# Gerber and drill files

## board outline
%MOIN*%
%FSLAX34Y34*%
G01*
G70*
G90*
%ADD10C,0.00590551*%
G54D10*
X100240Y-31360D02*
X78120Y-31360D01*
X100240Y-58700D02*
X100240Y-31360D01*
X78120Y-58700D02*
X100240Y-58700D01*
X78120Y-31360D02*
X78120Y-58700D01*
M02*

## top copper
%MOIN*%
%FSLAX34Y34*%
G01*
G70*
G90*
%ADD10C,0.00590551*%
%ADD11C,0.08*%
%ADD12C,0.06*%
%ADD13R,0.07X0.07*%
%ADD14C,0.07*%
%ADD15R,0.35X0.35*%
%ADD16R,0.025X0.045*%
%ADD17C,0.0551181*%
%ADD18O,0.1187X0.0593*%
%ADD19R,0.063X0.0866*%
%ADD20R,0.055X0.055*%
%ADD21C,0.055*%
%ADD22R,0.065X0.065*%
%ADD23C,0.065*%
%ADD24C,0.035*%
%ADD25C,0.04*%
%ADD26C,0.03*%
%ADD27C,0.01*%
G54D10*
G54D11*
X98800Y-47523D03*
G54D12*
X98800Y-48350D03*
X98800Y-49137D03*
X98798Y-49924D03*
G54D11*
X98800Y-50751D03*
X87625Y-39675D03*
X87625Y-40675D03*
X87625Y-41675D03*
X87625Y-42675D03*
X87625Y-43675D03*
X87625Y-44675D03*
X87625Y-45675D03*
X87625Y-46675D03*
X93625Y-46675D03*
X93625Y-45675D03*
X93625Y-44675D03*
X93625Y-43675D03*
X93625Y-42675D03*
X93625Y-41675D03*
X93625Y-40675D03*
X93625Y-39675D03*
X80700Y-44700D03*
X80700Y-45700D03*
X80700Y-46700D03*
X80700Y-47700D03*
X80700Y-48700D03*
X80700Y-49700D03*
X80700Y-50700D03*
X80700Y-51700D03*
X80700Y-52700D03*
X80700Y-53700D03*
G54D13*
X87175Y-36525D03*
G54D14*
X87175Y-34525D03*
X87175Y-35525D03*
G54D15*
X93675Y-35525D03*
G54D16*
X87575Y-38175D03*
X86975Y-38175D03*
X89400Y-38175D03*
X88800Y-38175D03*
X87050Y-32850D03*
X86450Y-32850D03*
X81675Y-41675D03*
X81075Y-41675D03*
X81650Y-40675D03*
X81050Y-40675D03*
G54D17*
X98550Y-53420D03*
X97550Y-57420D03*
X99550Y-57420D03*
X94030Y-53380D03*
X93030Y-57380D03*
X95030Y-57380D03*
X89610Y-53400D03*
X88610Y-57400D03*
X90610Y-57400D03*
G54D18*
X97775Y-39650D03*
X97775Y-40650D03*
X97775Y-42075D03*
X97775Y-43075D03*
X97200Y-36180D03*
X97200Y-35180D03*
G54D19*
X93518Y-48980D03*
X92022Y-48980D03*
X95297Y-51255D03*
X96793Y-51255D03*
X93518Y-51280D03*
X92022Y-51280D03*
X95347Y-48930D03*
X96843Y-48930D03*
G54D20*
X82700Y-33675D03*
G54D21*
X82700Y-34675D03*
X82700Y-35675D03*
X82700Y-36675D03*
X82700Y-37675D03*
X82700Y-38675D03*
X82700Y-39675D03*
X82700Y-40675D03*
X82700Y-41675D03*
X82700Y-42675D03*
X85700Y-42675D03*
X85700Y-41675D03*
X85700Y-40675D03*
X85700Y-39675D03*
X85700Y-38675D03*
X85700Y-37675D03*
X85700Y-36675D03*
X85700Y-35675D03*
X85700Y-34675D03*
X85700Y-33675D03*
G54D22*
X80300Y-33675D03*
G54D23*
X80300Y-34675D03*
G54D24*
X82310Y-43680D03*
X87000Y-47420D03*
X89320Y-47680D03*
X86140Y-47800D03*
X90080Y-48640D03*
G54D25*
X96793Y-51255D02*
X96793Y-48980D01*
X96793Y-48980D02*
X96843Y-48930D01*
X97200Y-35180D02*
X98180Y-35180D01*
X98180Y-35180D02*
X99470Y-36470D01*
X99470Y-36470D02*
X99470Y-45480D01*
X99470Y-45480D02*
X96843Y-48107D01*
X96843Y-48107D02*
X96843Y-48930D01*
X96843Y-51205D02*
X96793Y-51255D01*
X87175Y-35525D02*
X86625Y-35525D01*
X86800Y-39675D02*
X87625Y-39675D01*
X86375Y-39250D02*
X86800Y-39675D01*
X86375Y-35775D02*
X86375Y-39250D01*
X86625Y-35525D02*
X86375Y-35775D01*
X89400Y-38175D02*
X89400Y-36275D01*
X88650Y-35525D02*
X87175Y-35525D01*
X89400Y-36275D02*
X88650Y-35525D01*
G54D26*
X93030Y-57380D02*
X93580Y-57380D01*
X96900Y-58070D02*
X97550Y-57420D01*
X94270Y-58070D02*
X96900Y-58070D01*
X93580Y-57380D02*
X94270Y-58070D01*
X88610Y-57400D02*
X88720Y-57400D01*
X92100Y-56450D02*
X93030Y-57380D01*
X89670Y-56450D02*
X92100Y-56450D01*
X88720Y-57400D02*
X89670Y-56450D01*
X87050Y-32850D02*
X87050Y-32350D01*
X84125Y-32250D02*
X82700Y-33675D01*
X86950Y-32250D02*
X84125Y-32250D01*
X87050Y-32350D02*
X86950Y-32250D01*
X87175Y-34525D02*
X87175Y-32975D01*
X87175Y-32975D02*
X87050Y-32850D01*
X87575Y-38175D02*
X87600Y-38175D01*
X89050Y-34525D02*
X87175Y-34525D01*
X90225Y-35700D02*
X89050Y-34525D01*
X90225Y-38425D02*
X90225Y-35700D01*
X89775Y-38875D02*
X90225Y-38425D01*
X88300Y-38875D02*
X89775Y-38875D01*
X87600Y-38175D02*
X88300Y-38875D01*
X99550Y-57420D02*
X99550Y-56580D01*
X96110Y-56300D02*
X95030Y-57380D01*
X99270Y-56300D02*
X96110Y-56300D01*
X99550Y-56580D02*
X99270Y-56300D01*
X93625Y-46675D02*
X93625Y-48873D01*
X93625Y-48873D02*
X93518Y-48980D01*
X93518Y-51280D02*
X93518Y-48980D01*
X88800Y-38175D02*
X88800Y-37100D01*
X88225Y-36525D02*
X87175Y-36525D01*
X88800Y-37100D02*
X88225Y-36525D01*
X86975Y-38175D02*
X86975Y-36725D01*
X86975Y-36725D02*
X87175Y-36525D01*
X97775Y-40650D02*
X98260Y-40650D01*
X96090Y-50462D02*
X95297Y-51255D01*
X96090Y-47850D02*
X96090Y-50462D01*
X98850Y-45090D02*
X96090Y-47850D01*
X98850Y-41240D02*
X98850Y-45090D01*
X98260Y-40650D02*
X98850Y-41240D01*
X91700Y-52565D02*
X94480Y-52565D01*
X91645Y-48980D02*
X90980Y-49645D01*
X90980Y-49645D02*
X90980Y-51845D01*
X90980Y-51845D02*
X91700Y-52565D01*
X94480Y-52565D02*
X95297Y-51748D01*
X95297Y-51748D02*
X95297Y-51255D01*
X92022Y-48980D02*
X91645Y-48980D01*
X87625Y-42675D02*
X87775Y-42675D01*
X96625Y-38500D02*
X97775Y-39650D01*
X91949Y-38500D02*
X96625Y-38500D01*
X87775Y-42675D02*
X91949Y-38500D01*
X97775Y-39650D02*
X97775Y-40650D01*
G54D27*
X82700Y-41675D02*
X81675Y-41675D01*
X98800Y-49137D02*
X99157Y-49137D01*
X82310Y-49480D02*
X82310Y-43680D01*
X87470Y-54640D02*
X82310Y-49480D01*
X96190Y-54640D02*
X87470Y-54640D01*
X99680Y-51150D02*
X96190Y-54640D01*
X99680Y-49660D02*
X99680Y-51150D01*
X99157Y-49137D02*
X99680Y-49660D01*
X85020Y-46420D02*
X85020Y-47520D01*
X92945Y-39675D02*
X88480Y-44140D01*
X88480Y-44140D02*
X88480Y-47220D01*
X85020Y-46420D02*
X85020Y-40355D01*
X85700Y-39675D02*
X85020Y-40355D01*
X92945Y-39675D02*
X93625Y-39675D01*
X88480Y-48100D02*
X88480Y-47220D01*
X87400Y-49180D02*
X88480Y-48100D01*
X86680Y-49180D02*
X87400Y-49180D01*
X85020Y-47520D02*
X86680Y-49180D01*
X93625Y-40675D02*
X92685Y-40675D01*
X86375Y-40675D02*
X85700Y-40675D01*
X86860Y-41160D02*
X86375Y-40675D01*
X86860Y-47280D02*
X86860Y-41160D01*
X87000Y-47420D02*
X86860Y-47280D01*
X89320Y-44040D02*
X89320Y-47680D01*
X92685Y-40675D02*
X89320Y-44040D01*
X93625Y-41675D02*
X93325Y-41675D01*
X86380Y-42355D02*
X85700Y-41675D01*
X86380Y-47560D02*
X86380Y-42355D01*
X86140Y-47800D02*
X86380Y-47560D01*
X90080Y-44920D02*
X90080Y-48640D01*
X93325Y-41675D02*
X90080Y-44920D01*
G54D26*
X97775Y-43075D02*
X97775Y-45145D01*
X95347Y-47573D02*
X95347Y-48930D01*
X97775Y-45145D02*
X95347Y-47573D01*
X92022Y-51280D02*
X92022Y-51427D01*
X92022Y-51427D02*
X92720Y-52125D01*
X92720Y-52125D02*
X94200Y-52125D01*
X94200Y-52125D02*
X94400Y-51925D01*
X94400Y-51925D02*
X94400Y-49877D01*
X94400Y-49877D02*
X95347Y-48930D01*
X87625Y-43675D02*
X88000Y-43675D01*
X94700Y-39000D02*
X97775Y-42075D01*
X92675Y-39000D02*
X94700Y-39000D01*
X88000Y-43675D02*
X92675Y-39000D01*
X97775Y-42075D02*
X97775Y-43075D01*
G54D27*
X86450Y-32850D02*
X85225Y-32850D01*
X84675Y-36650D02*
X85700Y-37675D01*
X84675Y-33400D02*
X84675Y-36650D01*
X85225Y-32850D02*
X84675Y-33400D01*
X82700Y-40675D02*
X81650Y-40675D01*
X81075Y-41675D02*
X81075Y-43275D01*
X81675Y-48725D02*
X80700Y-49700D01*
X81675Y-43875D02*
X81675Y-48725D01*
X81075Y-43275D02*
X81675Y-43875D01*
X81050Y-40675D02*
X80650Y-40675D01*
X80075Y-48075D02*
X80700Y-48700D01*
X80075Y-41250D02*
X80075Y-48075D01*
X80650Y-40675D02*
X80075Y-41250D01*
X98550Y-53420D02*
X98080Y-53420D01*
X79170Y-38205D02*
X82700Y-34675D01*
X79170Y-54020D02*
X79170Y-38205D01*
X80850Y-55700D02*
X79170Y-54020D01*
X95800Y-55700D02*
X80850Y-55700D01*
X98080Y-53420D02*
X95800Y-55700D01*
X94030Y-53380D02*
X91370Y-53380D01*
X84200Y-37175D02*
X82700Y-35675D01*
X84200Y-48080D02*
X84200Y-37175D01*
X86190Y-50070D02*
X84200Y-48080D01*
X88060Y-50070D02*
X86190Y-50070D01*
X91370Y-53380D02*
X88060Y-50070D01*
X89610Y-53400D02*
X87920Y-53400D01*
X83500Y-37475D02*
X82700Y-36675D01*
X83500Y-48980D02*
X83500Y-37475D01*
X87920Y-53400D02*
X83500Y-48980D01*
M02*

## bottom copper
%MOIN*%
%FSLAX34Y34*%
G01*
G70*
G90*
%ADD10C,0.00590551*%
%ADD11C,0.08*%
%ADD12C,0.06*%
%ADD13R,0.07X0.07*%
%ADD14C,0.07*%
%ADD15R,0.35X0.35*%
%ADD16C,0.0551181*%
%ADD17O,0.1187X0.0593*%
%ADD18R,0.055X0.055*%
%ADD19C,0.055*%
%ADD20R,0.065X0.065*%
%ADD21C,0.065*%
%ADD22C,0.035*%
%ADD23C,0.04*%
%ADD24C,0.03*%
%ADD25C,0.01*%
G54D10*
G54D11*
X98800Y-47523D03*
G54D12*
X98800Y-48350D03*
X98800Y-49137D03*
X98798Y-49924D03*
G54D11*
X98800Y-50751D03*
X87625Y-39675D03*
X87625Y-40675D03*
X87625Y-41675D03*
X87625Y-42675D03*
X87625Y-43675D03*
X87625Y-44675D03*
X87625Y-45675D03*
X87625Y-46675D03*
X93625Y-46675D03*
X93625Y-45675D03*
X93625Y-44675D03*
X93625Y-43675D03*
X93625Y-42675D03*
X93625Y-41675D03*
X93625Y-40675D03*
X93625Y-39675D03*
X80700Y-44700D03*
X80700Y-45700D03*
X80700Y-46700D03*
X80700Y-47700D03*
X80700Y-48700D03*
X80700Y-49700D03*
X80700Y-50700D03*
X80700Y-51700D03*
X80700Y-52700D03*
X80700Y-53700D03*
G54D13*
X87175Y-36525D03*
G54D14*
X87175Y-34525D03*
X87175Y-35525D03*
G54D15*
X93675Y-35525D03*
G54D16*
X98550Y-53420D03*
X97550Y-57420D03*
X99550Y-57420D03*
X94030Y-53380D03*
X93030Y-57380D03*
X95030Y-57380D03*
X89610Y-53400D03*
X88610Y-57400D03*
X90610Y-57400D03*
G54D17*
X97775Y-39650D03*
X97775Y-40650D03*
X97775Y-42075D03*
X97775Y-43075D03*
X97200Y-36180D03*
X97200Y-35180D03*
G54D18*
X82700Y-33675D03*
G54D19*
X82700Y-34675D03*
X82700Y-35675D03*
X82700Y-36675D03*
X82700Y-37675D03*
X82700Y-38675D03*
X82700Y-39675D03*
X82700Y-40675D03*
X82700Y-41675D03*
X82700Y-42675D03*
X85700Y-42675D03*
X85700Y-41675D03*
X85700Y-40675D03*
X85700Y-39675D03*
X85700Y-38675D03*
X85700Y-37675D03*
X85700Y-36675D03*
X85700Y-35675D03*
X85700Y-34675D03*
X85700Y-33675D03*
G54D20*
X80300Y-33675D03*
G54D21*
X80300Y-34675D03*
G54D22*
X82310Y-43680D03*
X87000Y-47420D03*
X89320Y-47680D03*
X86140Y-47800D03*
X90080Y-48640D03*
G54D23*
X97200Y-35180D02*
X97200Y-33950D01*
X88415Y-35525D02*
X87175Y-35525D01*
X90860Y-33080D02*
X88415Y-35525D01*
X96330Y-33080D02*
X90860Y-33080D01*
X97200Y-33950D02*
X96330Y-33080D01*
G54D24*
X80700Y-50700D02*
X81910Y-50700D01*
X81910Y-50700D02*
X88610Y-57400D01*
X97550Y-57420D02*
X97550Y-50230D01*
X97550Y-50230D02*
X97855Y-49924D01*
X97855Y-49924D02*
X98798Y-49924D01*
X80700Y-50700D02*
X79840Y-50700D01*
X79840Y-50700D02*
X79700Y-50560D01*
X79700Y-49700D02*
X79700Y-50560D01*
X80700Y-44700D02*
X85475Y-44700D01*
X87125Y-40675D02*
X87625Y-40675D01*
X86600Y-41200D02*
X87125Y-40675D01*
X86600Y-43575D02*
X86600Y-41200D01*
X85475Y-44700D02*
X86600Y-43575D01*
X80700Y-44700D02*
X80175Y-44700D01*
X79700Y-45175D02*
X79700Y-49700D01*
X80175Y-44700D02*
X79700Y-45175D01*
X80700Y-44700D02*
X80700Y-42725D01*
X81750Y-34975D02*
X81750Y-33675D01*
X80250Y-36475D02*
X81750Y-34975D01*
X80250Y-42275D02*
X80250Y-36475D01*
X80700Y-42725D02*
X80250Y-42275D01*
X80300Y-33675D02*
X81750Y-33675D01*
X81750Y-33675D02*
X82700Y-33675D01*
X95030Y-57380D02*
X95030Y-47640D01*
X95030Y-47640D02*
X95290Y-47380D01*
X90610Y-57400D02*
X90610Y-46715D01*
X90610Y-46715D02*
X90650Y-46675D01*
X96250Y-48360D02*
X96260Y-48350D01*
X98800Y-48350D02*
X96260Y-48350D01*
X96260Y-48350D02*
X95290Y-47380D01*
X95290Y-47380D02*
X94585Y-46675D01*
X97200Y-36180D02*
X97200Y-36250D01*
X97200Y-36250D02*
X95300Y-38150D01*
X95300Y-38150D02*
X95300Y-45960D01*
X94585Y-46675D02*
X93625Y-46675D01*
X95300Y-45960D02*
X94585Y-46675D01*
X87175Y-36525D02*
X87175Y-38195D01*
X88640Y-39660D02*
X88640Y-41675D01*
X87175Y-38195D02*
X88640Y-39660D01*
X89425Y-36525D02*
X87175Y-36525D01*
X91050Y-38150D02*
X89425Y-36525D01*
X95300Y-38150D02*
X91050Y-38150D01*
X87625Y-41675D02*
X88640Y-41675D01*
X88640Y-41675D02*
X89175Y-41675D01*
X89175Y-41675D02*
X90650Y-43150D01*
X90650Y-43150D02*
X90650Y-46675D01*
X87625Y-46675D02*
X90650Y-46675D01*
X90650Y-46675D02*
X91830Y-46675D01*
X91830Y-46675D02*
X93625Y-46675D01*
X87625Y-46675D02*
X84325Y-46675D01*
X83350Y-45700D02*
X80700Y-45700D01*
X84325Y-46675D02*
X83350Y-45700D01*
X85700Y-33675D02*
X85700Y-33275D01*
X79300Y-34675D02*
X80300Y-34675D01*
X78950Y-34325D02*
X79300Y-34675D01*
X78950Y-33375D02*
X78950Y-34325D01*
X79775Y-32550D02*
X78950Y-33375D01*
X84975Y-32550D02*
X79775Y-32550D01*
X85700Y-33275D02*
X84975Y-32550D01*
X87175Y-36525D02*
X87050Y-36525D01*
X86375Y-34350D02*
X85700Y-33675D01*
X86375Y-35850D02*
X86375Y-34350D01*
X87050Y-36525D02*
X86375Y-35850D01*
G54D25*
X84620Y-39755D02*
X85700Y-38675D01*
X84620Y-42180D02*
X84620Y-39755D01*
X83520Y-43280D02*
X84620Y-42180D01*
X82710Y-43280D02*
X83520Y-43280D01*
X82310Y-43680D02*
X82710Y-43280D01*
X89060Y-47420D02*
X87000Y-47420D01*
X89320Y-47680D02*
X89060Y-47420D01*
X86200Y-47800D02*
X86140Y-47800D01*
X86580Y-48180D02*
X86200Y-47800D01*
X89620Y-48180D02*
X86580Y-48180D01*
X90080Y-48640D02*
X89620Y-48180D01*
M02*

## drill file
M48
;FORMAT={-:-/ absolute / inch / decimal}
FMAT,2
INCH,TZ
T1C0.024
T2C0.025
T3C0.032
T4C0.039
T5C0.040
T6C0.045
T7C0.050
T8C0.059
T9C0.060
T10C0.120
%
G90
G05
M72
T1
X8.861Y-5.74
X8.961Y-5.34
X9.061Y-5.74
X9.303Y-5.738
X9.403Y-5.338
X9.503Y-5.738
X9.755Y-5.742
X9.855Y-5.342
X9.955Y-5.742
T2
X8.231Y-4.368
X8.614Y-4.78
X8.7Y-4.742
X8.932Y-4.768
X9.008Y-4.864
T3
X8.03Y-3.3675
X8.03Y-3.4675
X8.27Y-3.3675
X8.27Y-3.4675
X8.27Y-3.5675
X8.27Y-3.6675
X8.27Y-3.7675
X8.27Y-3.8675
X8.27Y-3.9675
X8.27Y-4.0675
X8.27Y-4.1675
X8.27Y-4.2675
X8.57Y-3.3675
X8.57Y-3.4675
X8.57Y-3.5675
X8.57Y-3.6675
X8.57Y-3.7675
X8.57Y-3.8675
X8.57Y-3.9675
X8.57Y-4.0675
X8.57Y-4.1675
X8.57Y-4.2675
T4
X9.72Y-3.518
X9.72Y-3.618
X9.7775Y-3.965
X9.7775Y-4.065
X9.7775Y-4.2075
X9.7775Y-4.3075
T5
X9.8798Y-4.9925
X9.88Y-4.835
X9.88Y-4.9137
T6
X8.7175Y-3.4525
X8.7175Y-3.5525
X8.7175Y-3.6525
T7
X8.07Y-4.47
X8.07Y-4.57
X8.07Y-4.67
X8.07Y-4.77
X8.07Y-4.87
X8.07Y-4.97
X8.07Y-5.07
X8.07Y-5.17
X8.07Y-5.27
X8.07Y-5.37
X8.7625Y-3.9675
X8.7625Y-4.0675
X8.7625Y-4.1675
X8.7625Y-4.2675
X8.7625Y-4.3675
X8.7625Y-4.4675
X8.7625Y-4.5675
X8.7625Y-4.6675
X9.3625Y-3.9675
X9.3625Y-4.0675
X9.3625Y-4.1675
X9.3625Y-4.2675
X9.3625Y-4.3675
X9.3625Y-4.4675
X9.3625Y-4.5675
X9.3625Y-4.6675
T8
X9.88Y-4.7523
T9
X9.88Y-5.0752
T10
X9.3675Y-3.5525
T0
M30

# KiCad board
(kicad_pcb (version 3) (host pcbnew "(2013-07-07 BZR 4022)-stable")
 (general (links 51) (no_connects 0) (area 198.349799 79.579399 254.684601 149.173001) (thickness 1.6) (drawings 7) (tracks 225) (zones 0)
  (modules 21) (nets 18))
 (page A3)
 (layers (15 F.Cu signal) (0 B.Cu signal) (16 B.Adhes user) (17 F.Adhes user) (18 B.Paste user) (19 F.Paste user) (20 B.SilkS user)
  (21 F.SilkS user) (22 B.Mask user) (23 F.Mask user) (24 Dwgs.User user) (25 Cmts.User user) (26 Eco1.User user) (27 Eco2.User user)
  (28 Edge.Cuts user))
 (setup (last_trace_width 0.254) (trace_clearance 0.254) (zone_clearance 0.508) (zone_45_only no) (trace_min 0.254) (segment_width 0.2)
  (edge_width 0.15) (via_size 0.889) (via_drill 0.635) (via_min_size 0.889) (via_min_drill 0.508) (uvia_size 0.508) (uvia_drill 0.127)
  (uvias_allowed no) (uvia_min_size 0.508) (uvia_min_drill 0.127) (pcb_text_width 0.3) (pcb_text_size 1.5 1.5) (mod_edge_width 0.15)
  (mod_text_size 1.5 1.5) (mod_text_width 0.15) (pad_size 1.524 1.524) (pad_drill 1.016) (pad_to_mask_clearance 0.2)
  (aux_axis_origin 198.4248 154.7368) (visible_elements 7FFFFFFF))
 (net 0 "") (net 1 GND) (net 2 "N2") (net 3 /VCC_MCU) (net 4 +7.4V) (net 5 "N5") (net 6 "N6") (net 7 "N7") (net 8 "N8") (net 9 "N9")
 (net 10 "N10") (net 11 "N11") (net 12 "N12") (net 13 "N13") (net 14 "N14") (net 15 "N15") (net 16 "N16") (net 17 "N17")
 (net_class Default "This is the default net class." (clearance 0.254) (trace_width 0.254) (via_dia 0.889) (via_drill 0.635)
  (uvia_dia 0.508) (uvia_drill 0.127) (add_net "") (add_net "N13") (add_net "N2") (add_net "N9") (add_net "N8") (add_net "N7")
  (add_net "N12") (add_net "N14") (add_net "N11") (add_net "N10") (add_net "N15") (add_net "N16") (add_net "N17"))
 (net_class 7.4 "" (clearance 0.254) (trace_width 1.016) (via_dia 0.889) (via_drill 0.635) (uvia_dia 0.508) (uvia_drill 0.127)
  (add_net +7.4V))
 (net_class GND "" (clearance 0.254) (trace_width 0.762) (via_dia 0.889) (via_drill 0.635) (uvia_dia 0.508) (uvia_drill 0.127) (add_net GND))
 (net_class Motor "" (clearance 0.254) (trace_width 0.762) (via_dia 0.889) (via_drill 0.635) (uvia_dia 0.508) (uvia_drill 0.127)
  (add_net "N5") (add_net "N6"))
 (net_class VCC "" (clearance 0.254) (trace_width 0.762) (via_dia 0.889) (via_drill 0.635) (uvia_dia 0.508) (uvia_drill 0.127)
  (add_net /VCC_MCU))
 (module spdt (layer F.Cu) (at 250.952 122.809 270)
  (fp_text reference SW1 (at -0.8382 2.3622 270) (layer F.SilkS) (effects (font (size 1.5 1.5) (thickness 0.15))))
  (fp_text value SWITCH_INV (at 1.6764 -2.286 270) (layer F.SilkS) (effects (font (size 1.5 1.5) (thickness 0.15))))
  (pad 4 thru_hole circle (at -2.1 0 270) (size 2.032 2.032) (drill 1.4986) (layers *.Cu *.Mask F.SilkS))
  (pad 1 thru_hole circle (at 0 0 270) (size 1.524 1.524) (drill 1.016) (layers *.Cu *.Mask F.SilkS) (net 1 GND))
  (pad 2 thru_hole circle (at 2 0 270) (size 1.524 1.524) (drill 1.016) (layers *.Cu *.Mask F.SilkS) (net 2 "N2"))
  (pad 3 thru_hole circle (at 4 0.00508 270) (size 1.524 1.524) (drill 1.016) (layers *.Cu *.Mask F.SilkS) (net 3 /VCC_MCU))
  (pad 5 thru_hole circle (at 6.1 0 270) (size 2.032 2.032) (drill 1.524) (layers *.Cu *.Mask F.SilkS)))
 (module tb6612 (layer F.Cu) (at 233.6165 102.9335)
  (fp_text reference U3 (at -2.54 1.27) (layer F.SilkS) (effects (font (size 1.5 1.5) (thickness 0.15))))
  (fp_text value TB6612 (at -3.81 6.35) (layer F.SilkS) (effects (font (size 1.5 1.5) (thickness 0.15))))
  (pad 1 thru_hole circle (at -11.049 -2.159) (size 2.032 2.032) (drill 1.27) (layers *.Cu *.Mask F.SilkS) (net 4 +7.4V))
  (pad 2 thru_hole circle (at -11.049 0.381) (size 2.032 2.032) (drill 1.27) (layers *.Cu *.Mask F.SilkS) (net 3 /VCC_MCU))
  (pad 3 thru_hole circle (at -11.049 2.921) (size 2.032 2.032) (drill 1.27) (layers *.Cu *.Mask F.SilkS) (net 1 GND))
  (pad 4 thru_hole circle (at -11.049 5.461) (size 2.032 2.032) (drill 1.27) (layers *.Cu *.Mask F.SilkS) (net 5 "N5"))
  (pad 5 thru_hole circle (at -11.049 8.001) (size 2.032 2.032) (drill 1.27) (layers *.Cu *.Mask F.SilkS) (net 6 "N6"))
  (pad 6 thru_hole circle (at -11.049 10.541) (size 2.032 2.032) (drill 1.27) (layers *.Cu *.Mask F.SilkS))
  (pad 7 thru_hole circle (at -11.049 13.081) (size 2.032 2.032) (drill 1.27) (layers *.Cu *.Mask F.SilkS))
  (pad 8 thru_hole circle (at -11.049 15.621) (size 2.032 2.032) (drill 1.27) (layers *.Cu *.Mask F.SilkS) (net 1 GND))
  (pad 9 thru_hole circle (at 4.191 15.621) (size 2.032 2.032) (drill 1.27) (layers *.Cu *.Mask F.SilkS) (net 1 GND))
  (pad 10 thru_hole circle (at 4.191 13.081) (size 2.032 2.032) (drill 1.27) (layers *.Cu *.Mask F.SilkS))
  (pad 11 thru_hole circle (at 4.191 10.541) (size 2.032 2.032) (drill 1.27) (layers *.Cu *.Mask F.SilkS))
  (pad 12 thru_hole circle (at 4.191 8.001) (size 2.032 2.032) (drill 1.27) (layers *.Cu *.Mask F.SilkS))
  (pad 13 thru_hole circle (at 4.191 5.461) (size 2.032 2.032) (drill 1.27) (layers *.Cu *.Mask F.SilkS))
  (pad 14 thru_hole circle (at 4.191 2.921) (size 2.032 2.032) (drill 1.27) (layers *.Cu *.Mask F.SilkS) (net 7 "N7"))
  (pad 15 thru_hole circle (at 4.191 0.381) (size 2.032 2.032) (drill 1.27) (layers *.Cu *.Mask F.SilkS) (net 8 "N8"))
  (pad 16 thru_hole circle (at 4.191 -2.159) (size 2.032 2.032) (drill 1.27) (layers *.Cu *.Mask F.SilkS) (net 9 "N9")))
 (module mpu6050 (layer F.Cu) (at 204.978 124.968)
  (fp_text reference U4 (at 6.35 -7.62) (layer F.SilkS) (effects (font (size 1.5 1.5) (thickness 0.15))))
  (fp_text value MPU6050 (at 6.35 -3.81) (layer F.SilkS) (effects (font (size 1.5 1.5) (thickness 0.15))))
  (pad 1 thru_hole circle (at 0 -11.43) (size 2.032 2.032) (drill 1.27) (layers *.Cu *.Mask F.SilkS) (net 3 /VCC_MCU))
  (pad 2 thru_hole circle (at 0 -8.89) (size 2.032 2.032) (drill 1.27) (layers *.Cu *.Mask F.SilkS) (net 1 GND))
  (pad 3 thru_hole circle (at 0 -6.35) (size 2.032 2.032) (drill 1.27) (layers *.Cu *.Mask F.SilkS))
  (pad 4 thru_hole circle (at 0 -3.81) (size 2.032 2.032) (drill 1.27) (layers *.Cu *.Mask F.SilkS))
  (pad 5 thru_hole circle (at 0 -1.27) (size 2.032 2.032) (drill 1.27) (layers *.Cu *.Mask F.SilkS) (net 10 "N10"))
  (pad 6 thru_hole circle (at 0 1.27) (size 2.032 2.032) (drill 1.27) (layers *.Cu *.Mask F.SilkS) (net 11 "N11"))
  (pad 7 thru_hole circle (at 0 3.81) (size 2.032 2.032) (drill 1.27) (layers *.Cu *.Mask F.SilkS) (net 3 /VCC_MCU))
  (pad 8 thru_hole circle (at 0 6.35) (size 2.032 2.032) (drill 1.27) (layers *.Cu *.Mask F.SilkS))
  (pad 9 thru_hole circle (at 0 8.89) (size 2.032 2.032) (drill 1.27) (layers *.Cu *.Mask F.SilkS))
  (pad 10 thru_hole circle (at 0 11.43) (size 2.032 2.032) (drill 1.27) (layers *.Cu *.Mask F.SilkS)))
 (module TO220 (layer F.Cu) (at 221.4245 90.2335)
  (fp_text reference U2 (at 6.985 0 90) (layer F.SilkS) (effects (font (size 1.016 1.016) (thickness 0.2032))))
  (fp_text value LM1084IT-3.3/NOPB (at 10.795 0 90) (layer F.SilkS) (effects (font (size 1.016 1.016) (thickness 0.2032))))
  (pad 1 thru_hole rect (at 0 2.54) (size 1.778 1.778) (drill 1.143) (layers *.Cu *.Mask F.SilkS) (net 1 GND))
  (pad 2 thru_hole circle (at 0 -2.54) (size 1.778 1.778) (drill 1.143) (layers *.Cu *.Mask F.SilkS) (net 3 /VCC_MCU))
  (pad 3 thru_hole circle (at 0 0) (size 1.778 1.778) (drill 1.143) (layers *.Cu *.Mask F.SilkS) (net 4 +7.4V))
  (pad 4 thru_hole rect (at 16.51 0) (size 8.89 8.89) (drill 3.048) (layers *.Cu *.SilkS *.Mask)))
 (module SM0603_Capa (layer F.Cu) (at 221.6785 96.9645 180)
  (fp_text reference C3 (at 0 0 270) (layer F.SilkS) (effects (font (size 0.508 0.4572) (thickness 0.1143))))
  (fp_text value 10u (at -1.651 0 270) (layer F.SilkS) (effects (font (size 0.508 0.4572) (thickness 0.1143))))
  (pad 1 smd rect (at -0.762 0 180) (size 0.635 1.143) (layers F.Cu F.Paste F.Mask) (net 3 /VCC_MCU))
  (pad 2 smd rect (at 0.762 0 180) (size 0.635 1.143) (layers F.Cu F.Paste F.Mask) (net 1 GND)))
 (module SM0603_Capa (layer F.Cu) (at 226.314 96.9645 180)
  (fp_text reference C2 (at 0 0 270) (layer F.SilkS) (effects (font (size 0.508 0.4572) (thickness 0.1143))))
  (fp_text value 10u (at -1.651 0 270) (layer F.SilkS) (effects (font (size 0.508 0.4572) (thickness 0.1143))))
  (pad 1 smd rect (at -0.762 0 180) (size 0.635 1.143) (layers F.Cu F.Paste F.Mask) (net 4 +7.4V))
  (pad 2 smd rect (at 0.762 0 180) (size 0.635 1.143) (layers F.Cu F.Paste F.Mask) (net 1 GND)))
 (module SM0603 (layer F.Cu) (at 220.345 83.439 180)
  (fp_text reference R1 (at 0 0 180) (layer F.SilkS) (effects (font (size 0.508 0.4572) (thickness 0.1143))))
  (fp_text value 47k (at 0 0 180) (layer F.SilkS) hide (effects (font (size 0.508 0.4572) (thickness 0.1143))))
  (pad 1 smd rect (at -0.762 0 180) (size 0.635 1.143) (layers F.Cu F.Paste F.Mask) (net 3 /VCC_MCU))
  (pad 2 smd rect (at 0.762 0 180) (size 0.635 1.143) (layers F.Cu F.Paste F.Mask) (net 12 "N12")))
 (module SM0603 (layer F.Cu) (at 206.6925 105.8545 180)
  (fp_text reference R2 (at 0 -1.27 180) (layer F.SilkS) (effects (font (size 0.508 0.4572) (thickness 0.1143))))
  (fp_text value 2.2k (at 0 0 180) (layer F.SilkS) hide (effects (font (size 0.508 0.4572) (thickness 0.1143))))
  (pad 1 smd rect (at -0.762 0 180) (size 0.635 1.143) (layers F.Cu F.Paste F.Mask) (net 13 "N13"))
  (pad 2 smd rect (at 0.762 0 180) (size 0.635 1.143) (layers F.Cu F.Paste F.Mask) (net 11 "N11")))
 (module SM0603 (layer F.Cu) (at 206.629 103.3145 180)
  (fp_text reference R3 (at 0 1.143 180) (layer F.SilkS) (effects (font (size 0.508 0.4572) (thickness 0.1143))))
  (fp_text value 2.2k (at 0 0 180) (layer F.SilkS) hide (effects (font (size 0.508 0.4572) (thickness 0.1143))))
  (pad 1 smd rect (at -0.762 0 180) (size 0.635 1.143) (layers F.Cu F.Paste F.Mask) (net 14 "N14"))
  (pad 2 smd rect (at 0.762 0 180) (size 0.635 1.143) (layers F.Cu F.Paste F.Mask) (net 10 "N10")))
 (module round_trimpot (layer F.Cu) (at 250.317 145.8468)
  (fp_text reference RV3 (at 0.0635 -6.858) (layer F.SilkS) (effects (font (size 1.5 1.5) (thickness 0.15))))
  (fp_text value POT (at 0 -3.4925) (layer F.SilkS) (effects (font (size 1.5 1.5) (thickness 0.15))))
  (pad 2 thru_hole circle (at 0 -10.16) (size 1.4 1.4) (drill 0.6) (layers *.Cu *.Mask F.SilkS) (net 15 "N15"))
  (pad 1 thru_hole circle (at -2.54 0) (size 1.4 1.4) (drill 0.6) (layers *.Cu *.Mask F.SilkS) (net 3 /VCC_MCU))
  (pad 3 thru_hole circle (at 2.54 0) (size 1.4 1.4) (drill 0.6) (layers *.Cu *.Mask F.SilkS) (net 1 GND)))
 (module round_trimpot (layer F.Cu) (at 238.8362 145.7452)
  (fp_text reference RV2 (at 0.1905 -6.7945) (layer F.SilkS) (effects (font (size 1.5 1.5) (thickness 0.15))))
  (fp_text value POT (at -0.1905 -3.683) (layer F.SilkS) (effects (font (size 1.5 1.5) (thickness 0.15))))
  (pad 2 thru_hole circle (at 0 -10.16) (size 1.4 1.4) (drill 0.6) (layers *.Cu *.Mask F.SilkS) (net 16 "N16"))
  (pad 1 thru_hole circle (at -2.54 0) (size 1.4 1.4) (drill 0.6) (layers *.Cu *.Mask F.SilkS) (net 3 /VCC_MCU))
  (pad 3 thru_hole circle (at 2.54 0) (size 1.4 1.4) (drill 0.6) (layers *.Cu *.Mask F.SilkS) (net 1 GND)))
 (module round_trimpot (layer F.Cu) (at 227.6094 145.796)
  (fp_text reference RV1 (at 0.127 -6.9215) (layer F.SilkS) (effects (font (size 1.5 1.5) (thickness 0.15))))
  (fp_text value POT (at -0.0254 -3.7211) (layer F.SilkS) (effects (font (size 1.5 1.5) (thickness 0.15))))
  (pad 2 thru_hole circle (at 0 -10.16) (size 1.4 1.4) (drill 0.6) (layers *.Cu *.Mask F.SilkS) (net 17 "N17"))
  (pad 1 thru_hole circle (at -2.54 0) (size 1.4 1.4) (drill 0.6) (layers *.Cu *.Mask F.SilkS) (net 3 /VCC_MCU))
  (pad 3 thru_hole circle (at 2.54 0) (size 1.4 1.4) (drill 0.6) (layers *.Cu *.Mask F.SilkS) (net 1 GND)))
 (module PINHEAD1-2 (layer F.Cu) (at 248.3485 101.981 270)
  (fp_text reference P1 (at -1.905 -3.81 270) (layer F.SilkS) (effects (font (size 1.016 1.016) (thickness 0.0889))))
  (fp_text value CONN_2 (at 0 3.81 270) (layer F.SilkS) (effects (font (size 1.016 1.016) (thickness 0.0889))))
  (pad 1 thru_hole oval (at -1.27 0 270) (size 1.50622 3.01498) (drill 0.99822) (layers *.Cu F.Paste F.SilkS F.Mask) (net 5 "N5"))
  (pad 2 thru_hole oval (at 1.27 0 270) (size 1.50622 3.01498) (drill 0.99822) (layers *.Cu F.Paste F.SilkS F.Mask) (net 5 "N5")))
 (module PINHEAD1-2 (layer F.Cu) (at 248.3485 108.1405 270)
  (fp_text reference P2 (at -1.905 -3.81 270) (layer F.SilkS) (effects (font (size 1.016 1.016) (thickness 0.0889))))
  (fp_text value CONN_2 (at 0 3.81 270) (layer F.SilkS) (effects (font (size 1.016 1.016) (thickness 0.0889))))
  (pad 1 thru_hole oval (at -1.27 0 270) (size 1.50622 3.01498) (drill 0.99822) (layers *.Cu F.Paste F.SilkS F.Mask) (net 6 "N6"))
  (pad 2 thru_hole oval (at 1.27 0 270) (size 1.50622 3.01498) (drill 0.99822) (layers *.Cu F.Paste F.SilkS F.Mask) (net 6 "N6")))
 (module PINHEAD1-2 (layer F.Cu) (at 246.888 90.6272 90)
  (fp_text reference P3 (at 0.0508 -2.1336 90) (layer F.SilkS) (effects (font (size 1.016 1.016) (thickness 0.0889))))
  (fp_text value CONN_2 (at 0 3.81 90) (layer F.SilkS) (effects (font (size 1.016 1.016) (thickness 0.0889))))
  (pad 1 thru_hole oval (at -1.27 0 90) (size 1.50622 3.01498) (drill 0.99822) (layers *.Cu F.Paste F.SilkS F.Mask) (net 1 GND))
  (pad 2 thru_hole oval (at 1.27 0 90) (size 1.50622 3.01498) (drill 0.99822) (layers *.Cu F.Paste F.SilkS F.Mask) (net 4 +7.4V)))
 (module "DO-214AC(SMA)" (layer F.Cu) (at 235.6358 124.4092 180)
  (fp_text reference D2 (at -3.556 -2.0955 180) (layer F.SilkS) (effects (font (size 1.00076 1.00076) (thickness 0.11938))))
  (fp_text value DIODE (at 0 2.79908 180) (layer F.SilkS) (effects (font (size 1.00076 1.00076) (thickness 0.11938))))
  (pad 1 smd rect (at -1.89992 0 180) (size 1.6002 2.19964) (layers F.Cu F.Paste F.Mask) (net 1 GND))
  (pad 2 smd rect (at 1.89992 0 180) (size 1.6002 2.19964) (layers F.Cu F.Paste F.Mask) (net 5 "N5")))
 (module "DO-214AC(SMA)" (layer F.Cu) (at 243.9543 130.1877)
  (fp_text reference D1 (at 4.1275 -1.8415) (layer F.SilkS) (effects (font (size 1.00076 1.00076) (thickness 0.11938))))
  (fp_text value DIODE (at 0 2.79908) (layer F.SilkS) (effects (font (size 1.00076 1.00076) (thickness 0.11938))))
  (pad 1 smd rect (at -1.89992 0) (size 1.6002 2.19964) (layers F.Cu F.Paste F.Mask) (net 5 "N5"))
  (pad 2 smd rect (at 1.89992 0) (size 1.6002 2.19964) (layers F.Cu F.Paste F.Mask) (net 4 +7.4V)))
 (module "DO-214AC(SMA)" (layer F.Cu) (at 235.6358 130.2512 180)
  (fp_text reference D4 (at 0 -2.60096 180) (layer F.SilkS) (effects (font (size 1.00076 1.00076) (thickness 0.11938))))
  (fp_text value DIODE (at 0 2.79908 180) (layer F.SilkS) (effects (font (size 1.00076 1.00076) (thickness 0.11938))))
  (pad 1 smd rect (at -1.89992 0 180) (size 1.6002 2.19964) (layers F.Cu F.Paste F.Mask) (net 1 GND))
  (pad 2 smd rect (at 1.89992 0 180) (size 1.6002 2.19964) (layers F.Cu F.Paste F.Mask) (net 6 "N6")))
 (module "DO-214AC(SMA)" (layer F.Cu) (at 244.0813 124.2822)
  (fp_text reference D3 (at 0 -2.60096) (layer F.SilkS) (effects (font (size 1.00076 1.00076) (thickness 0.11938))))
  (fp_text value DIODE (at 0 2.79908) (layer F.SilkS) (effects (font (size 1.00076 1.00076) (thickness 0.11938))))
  (pad 1 smd rect (at -1.89992 0) (size 1.6002 2.19964) (layers F.Cu F.Paste F.Mask) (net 6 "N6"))
  (pad 2 smd rect (at 1.89992 0) (size 1.6002 2.19964) (layers F.Cu F.Paste F.Mask) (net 4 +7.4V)))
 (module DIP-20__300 (layer F.Cu) (at 213.868 96.9645 270)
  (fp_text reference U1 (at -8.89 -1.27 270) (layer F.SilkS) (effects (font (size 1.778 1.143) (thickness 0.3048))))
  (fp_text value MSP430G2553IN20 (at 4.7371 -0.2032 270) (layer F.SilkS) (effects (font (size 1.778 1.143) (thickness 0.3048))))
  (pad 1 thru_hole rect (at -11.43 3.81 270) (size 1.397 1.397) (drill 0.8128) (layers *.Cu *.Mask F.SilkS) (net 3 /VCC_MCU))
  (pad 2 thru_hole circle (at -8.89 3.81 270) (size 1.397 1.397) (drill 0.8128) (layers *.Cu *.Mask F.SilkS) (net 15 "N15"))
  (pad 3 thru_hole circle (at -6.35 3.81 270) (size 1.397 1.397) (drill 0.8128) (layers *.Cu *.Mask F.SilkS) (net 16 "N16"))
  (pad 4 thru_hole circle (at -3.81 3.81 270) (size 1.397 1.397) (drill 0.8128) (layers *.Cu *.Mask F.SilkS) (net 17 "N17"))
  (pad 5 thru_hole circle (at -1.27 3.81 270) (size 1.397 1.397) (drill 0.8128) (layers *.Cu *.Mask F.SilkS))
  (pad 6 thru_hole circle (at 1.27 3.81 270) (size 1.397 1.397) (drill 0.8128) (layers *.Cu *.Mask F.SilkS))
  (pad 7 thru_hole circle (at 3.81 3.81 270) (size 1.397 1.397) (drill 0.8128) (layers *.Cu *.Mask F.SilkS))
  (pad 8 thru_hole circle (at 6.35 3.81 270) (size 1.397 1.397) (drill 0.8128) (layers *.Cu *.Mask F.SilkS) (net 14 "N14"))
  (pad 9 thru_hole circle (at 8.89 3.81 270) (size 1.397 1.397) (drill 0.8128) (layers *.Cu *.Mask F.SilkS) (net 13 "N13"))
  (pad 10 thru_hole circle (at 11.43 3.81 270) (size 1.397 1.397) (drill 0.8128) (layers *.Cu *.Mask F.SilkS))
  (pad 11 thru_hole circle (at 11.43 -3.81 270) (size 1.397 1.397) (drill 0.8128) (layers *.Cu *.Mask F.SilkS))
  (pad 12 thru_hole circle (at 8.89 -3.81 270) (size 1.397 1.397) (drill 0.8128) (layers *.Cu *.Mask F.SilkS) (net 7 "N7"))
  (pad 13 thru_hole circle (at 6.35 -3.81 270) (size 1.397 1.397) (drill 0.8128) (layers *.Cu *.Mask F.SilkS) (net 8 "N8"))
  (pad 14 thru_hole circle (at 3.81 -3.81 270) (size 1.397 1.397) (drill 0.8128) (layers *.Cu *.Mask F.SilkS) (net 9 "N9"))
  (pad 15 thru_hole circle (at 1.27 -3.81 270) (size 1.397 1.397) (drill 0.8128) (layers *.Cu *.Mask F.SilkS) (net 2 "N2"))
  (pad 16 thru_hole circle (at -1.27 -3.81 270) (size 1.397 1.397) (drill 0.8128) (layers *.Cu *.Mask F.SilkS) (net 12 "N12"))
  (pad 17 thru_hole circle (at -3.81 -3.81 270) (size 1.397 1.397) (drill 0.8128) (layers *.Cu *.Mask F.SilkS))
  (pad 18 thru_hole circle (at -6.35 -3.81 270) (size 1.397 1.397) (drill 0.8128) (layers *.Cu *.Mask F.SilkS))
  (pad 19 thru_hole circle (at -8.89 -3.81 270) (size 1.397 1.397) (drill 0.8128) (layers *.Cu *.Mask F.SilkS))
  (pad 20 thru_hole circle (at -11.43 -3.81 270) (size 1.397 1.397) (drill 0.8128) (layers *.Cu *.Mask F.SilkS) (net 1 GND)))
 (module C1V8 (layer F.Cu) (at 203.962 86.8045 270)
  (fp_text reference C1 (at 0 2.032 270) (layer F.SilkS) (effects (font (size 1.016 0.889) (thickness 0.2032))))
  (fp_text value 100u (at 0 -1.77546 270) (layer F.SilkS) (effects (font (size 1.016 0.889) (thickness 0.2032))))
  (pad 1 thru_hole rect (at -1.27 0 270) (size 1.651 1.651) (drill 0.8128) (layers *.Cu *.Mask F.SilkS) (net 3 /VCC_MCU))
  (pad 2 thru_hole circle (at 1.27 0 270) (size 1.651 1.651) (drill 0.8128) (layers *.Cu *.Mask F.SilkS) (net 1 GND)))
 (gr_line (start 254.6096 79.6544) (end 198.4248 79.6544) (angle 90) (layer Edge.Cuts) (width 0.15))
 (gr_line (start 254.6096 149.098) (end 254.6096 79.6544) (angle 90) (layer Edge.Cuts) (width 0.15))
 (gr_line (start 198.4248 149.098) (end 254.6096 149.098) (angle 90) (layer Edge.Cuts) (width 0.15))
 (gr_line (start 198.4248 79.6544) (end 198.4248 149.098) (angle 90) (layer Edge.Cuts) (width 0.15))
 (segment (start 245.85422 130.1877) (end 245.85422 124.4092) (width 1.016) (layer F.Cu) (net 4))
 (segment (start 245.85422 124.4092) (end 245.98122 124.2822) (width 1.016) (layer F.Cu) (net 4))
 (segment (start 246.888 89.3572) (end 249.3772 89.3572) (width 1.016) (layer F.Cu) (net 4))
 (segment (start 249.3772 89.3572) (end 252.6538 92.6338) (width 1.016) (layer F.Cu) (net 4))
 (segment (start 252.6538 92.6338) (end 252.6538 115.5192) (width 1.016) (layer F.Cu) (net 4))
 (segment (start 252.6538 115.5192) (end 245.98122 122.19178) (width 1.016) (layer F.Cu) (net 4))
 (segment (start 245.98122 122.19178) (end 245.98122 124.2822) (width 1.016) (layer F.Cu) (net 4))
 (segment (start 246.888 89.3572) (end 246.888 86.233) (width 1.016) (layer B.Cu) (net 4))
 (segment (start 224.5741 90.2335) (end 221.4245 90.2335) (width 1.016) (layer B.Cu) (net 4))
 (segment (start 230.7844 84.0232) (end 224.5741 90.2335) (width 1.016) (layer B.Cu) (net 4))
 (segment (start 244.6782 84.0232) (end 230.7844 84.0232) (width 1.016) (layer B.Cu) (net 4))
 (segment (start 246.888 86.233) (end 244.6782 84.0232) (width 1.016) (layer B.Cu) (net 4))
 (segment (start 245.98122 130.0607) (end 245.85422 130.1877) (width 1.016) (layer F.Cu) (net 4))
 (segment (start 221.4245 90.2335) (end 220.0275 90.2335) (width 1.016) (layer F.Cu) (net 4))
 (segment (start 220.472 100.7745) (end 222.5675 100.7745) (width 1.016) (layer F.Cu) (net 4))
 (segment (start 219.3925 99.695) (end 220.472 100.7745) (width 1.016) (layer F.Cu) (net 4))
 (segment (start 219.3925 90.8685) (end 219.3925 99.695) (width 1.016) (layer F.Cu) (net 4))
 (segment (start 220.0275 90.2335) (end 219.3925 90.8685) (width 1.016) (layer F.Cu) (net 4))
 (segment (start 227.076 96.9645) (end 227.076 92.1385) (width 1.016) (layer F.Cu) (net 4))
 (segment (start 225.171 90.2335) (end 221.4245 90.2335) (width 1.016) (layer F.Cu) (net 4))
 (segment (start 227.076 92.1385) (end 225.171 90.2335) (width 1.016) (layer F.Cu) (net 4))
 (segment (start 236.2962 145.7452) (end 237.6932 145.7452) (width 0.762) (layer F.Cu) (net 3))
 (segment (start 246.126 147.4978) (end 247.777 145.8468) (width 0.762) (layer F.Cu) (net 3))
 (segment (start 239.4458 147.4978) (end 246.126 147.4978) (width 0.762) (layer F.Cu) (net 3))
 (segment (start 237.6932 145.7452) (end 239.4458 147.4978) (width 0.762) (layer F.Cu) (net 3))
 (segment (start 225.0694 145.796) (end 225.3488 145.796) (width 0.762) (layer F.Cu) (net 3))
 (segment (start 233.934 143.383) (end 236.2962 145.7452) (width 0.762) (layer F.Cu) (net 3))
 (segment (start 227.7618 143.383) (end 233.934 143.383) (width 0.762) (layer F.Cu) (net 3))
 (segment (start 225.3488 145.796) (end 227.7618 143.383) (width 0.762) (layer F.Cu) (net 3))
 (segment (start 204.978 128.778) (end 208.0514 128.778) (width 0.762) (layer B.Cu) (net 3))
 (segment (start 208.0514 128.778) (end 225.0694 145.796) (width 0.762) (layer B.Cu) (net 3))
 (segment (start 247.777 145.8468) (end 247.777 127.5842) (width 0.762) (layer B.Cu) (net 3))
 (segment (start 247.777 127.5842) (end 248.5522 126.809) (width 0.762) (layer B.Cu) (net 3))
 (segment (start 248.5522 126.809) (end 250.94692 126.809) (width 0.762) (layer B.Cu) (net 3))
 (segment (start 204.978 128.778) (end 202.7936 128.778) (width 0.762) (layer B.Cu) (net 3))
 (segment (start 202.7936 128.778) (end 202.438 128.4224) (width 0.762) (layer B.Cu) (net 3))
 (segment (start 202.438 126.238) (end 202.438 128.4224) (width 0.762) (layer B.Cu) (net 3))
 (segment (start 204.978 113.538) (end 217.1065 113.538) (width 0.762) (layer B.Cu) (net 3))
 (segment (start 221.2975 103.3145) (end 222.5675 103.3145) (width 0.762) (layer B.Cu) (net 3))
 (segment (start 219.964 104.648) (end 221.2975 103.3145) (width 0.762) (layer B.Cu) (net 3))
 (segment (start 219.964 110.6805) (end 219.964 104.648) (width 0.762) (layer B.Cu) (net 3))
 (segment (start 217.1065 113.538) (end 219.964 110.6805) (width 0.762) (layer B.Cu) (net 3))
 (segment (start 204.978 113.538) (end 203.6445 113.538) (width 0.762) (layer B.Cu) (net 3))
 (segment (start 202.438 114.7445) (end 202.438 126.238) (width 0.762) (layer B.Cu) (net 3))
 (segment (start 203.6445 113.538) (end 202.438 114.7445) (width 0.762) (layer B.Cu) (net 3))
 (segment (start 204.978 113.538) (end 204.978 108.5215) (width 0.762) (layer B.Cu) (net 3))
 (segment (start 207.645 88.8365) (end 207.645 85.5345) (width 0.762) (layer B.Cu) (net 3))
 (segment (start 203.835 92.6465) (end 207.645 88.8365) (width 0.762) (layer B.Cu) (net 3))
 (segment (start 203.835 107.3785) (end 203.835 92.6465) (width 0.762) (layer B.Cu) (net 3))
 (segment (start 204.978 108.5215) (end 203.835 107.3785) (width 0.762) (layer B.Cu) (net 3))
 (segment (start 221.107 83.439) (end 221.107 82.169) (width 0.762) (layer F.Cu) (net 3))
 (segment (start 213.6775 81.915) (end 210.058 85.5345) (width 0.762) (layer F.Cu) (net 3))
 (segment (start 220.853 81.915) (end 213.6775 81.915) (width 0.762) (layer F.Cu) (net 3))
 (segment (start 221.107 82.169) (end 220.853 81.915) (width 0.762) (layer F.Cu) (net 3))
 (segment (start 203.962 85.5345) (end 207.645 85.5345) (width 0.762) (layer B.Cu) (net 3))
 (segment (start 207.645 85.5345) (end 210.058 85.5345) (width 0.762) (layer B.Cu) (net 3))
 (segment (start 221.4245 87.6935) (end 221.4245 83.7565) (width 0.762) (layer F.Cu) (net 3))
 (segment (start 221.4245 83.7565) (end 221.107 83.439) (width 0.762) (layer F.Cu) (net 3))
 (segment (start 222.4405 96.9645) (end 222.504 96.9645) (width 0.762) (layer F.Cu) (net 3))
 (segment (start 226.187 87.6935) (end 221.4245 87.6935) (width 0.762) (layer F.Cu) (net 3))
 (segment (start 229.1715 90.678) (end 226.187 87.6935) (width 0.762) (layer F.Cu) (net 3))
 (segment (start 229.1715 97.5995) (end 229.1715 90.678) (width 0.762) (layer F.Cu) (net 3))
 (segment (start 228.0285 98.7425) (end 229.1715 97.5995) (width 0.762) (layer F.Cu) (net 3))
 (segment (start 224.282 98.7425) (end 228.0285 98.7425) (width 0.762) (layer F.Cu) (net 3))
 (segment (start 222.504 96.9645) (end 224.282 98.7425) (width 0.762) (layer F.Cu) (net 3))
 (segment (start 252.857 145.8468) (end 252.857 143.7132) (width 0.762) (layer F.Cu) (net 1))
 (segment (start 244.1194 143.002) (end 241.3762 145.7452) (width 0.762) (layer F.Cu) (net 1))
 (segment (start 252.1458 143.002) (end 244.1194 143.002) (width 0.762) (layer F.Cu) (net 1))
 (segment (start 252.857 143.7132) (end 252.1458 143.002) (width 0.762) (layer F.Cu) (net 1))
 (segment (start 241.3762 145.7452) (end 241.3762 121.0056) (width 0.762) (layer B.Cu) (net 1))
 (segment (start 241.3762 121.0056) (end 242.0366 120.3452) (width 0.762) (layer B.Cu) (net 1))
 (segment (start 230.1494 145.796) (end 230.1494 118.6561) (width 0.762) (layer B.Cu) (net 1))
 (segment (start 230.1494 118.6561) (end 230.251 118.5545) (width 0.762) (layer B.Cu) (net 1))
 (segment (start 244.475 122.8344) (end 244.5004 122.809) (width 0.762) (layer B.Cu) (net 1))
 (segment (start 250.952 122.809) (end 244.5004 122.809) (width 0.762) (layer B.Cu) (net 1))
 (segment (start 244.5004 122.809) (end 242.0366 120.3452) (width 0.762) (layer B.Cu) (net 1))
 (segment (start 242.0366 120.3452) (end 240.2459 118.5545) (width 0.762) (layer B.Cu) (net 1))
 (segment (start 246.888 91.8972) (end 246.888 92.075) (width 0.762) (layer B.Cu) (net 1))
 (segment (start 246.888 92.075) (end 242.062 96.901) (width 0.762) (layer B.Cu) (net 1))
 (segment (start 237.8075 118.5545) (end 237.8075 124.13742) (width 0.762) (layer F.Cu) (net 1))
 (segment (start 237.8075 124.13742) (end 237.53572 124.4092) (width 0.762) (layer F.Cu) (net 1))
 (segment (start 242.062 96.901) (end 242.062 116.7384) (width 0.762) (layer B.Cu) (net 1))
 (segment (start 240.2459 118.5545) (end 237.8075 118.5545) (width 0.762) (layer B.Cu) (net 1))
 (segment (start 242.062 116.7384) (end 240.2459 118.5545) (width 0.762) (layer B.Cu) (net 1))
 (segment (start 221.4245 92.7735) (end 221.4245 97.0153) (width 0.762) (layer B.Cu) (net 1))
 (segment (start 225.1456 100.7364) (end 225.1456 105.8545) (width 0.762) (layer B.Cu) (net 1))
 (segment (start 221.4245 97.0153) (end 225.1456 100.7364) (width 0.762) (layer B.Cu) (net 1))
 (segment (start 237.53572 130.2512) (end 237.53572 124.4092) (width 0.762) (layer F.Cu) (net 1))
 (segment (start 227.1395 92.7735) (end 221.4245 92.7735) (width 0.762) (layer B.Cu) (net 1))
 (segment (start 231.267 96.901) (end 227.1395 92.7735) (width 0.762) (layer B.Cu) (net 1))
 (segment (start 242.062 96.901) (end 231.267 96.901) (width 0.762) (layer B.Cu) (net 1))
 (segment (start 222.5675 105.8545) (end 225.1456 105.8545) (width 0.762) (layer B.Cu) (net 1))
 (segment (start 225.1456 105.8545) (end 226.5045 105.8545) (width 0.762) (layer B.Cu) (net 1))
 (segment (start 226.5045 105.8545) (end 230.251 109.601) (width 0.762) (layer B.Cu) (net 1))
 (segment (start 230.251 109.601) (end 230.251 118.5545) (width 0.762) (layer B.Cu) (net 1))
 (segment (start 222.5675 118.5545) (end 230.251 118.5545) (width 0.762) (layer B.Cu) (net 1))
 (segment (start 230.251 118.5545) (end 233.2482 118.5545) (width 0.762) (layer B.Cu) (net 1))
 (segment (start 233.2482 118.5545) (end 237.8075 118.5545) (width 0.762) (layer B.Cu) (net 1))
 (segment (start 222.5675 118.5545) (end 214.1855 118.5545) (width 0.762) (layer B.Cu) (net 1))
 (segment (start 211.709 116.078) (end 204.978 116.078) (width 0.762) (layer B.Cu) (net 1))
 (segment (start 214.1855 118.5545) (end 211.709 116.078) (width 0.762) (layer B.Cu) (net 1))
 (segment (start 217.678 85.5345) (end 217.678 84.5185) (width 0.762) (layer B.Cu) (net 1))
 (segment (start 201.422 88.0745) (end 203.962 88.0745) (width 0.762) (layer B.Cu) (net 1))
 (segment (start 200.533 87.1855) (end 201.422 88.0745) (width 0.762) (layer B.Cu) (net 1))
 (segment (start 200.533 84.7725) (end 200.533 87.1855) (width 0.762) (layer B.Cu) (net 1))
 (segment (start 202.6285 82.677) (end 200.533 84.7725) (width 0.762) (layer B.Cu) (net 1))
 (segment (start 215.8365 82.677) (end 202.6285 82.677) (width 0.762) (layer B.Cu) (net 1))
 (segment (start 217.678 84.5185) (end 215.8365 82.677) (width 0.762) (layer B.Cu) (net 1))
 (segment (start 221.4245 92.7735) (end 221.107 92.7735) (width 0.762) (layer B.Cu) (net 1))
 (segment (start 219.3925 87.249) (end 217.678 85.5345) (width 0.762) (layer B.Cu) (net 1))
 (segment (start 219.3925 91.059) (end 219.3925 87.249) (width 0.762) (layer B.Cu) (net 1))
 (segment (start 221.107 92.7735) (end 219.3925 91.059) (width 0.762) (layer B.Cu) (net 1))
 (segment (start 225.552 96.9645) (end 225.552 94.234) (width 0.762) (layer F.Cu) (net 1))
 (segment (start 224.0915 92.7735) (end 221.4245 92.7735) (width 0.762) (layer F.Cu) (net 1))
 (segment (start 225.552 94.234) (end 224.0915 92.7735) (width 0.762) (layer F.Cu) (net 1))
 (segment (start 220.9165 96.9645) (end 220.9165 93.2815) (width 0.762) (layer F.Cu) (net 1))
 (segment (start 220.9165 93.2815) (end 221.4245 92.7735) (width 0.762) (layer F.Cu) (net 1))
 (segment (start 248.3485 103.251) (end 249.5804 103.251) (width 0.762) (layer F.Cu) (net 5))
 (segment (start 244.0686 128.17348) (end 242.05438 130.1877) (width 0.762) (layer F.Cu) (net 5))
 (segment (start 244.0686 121.539) (end 244.0686 128.17348) (width 0.762) (layer F.Cu) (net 5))
 (segment (start 251.079 114.5286) (end 244.0686 121.539) (width 0.762) (layer F.Cu) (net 5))
 (segment (start 251.079 104.7496) (end 251.079 114.5286) (width 0.762) (layer F.Cu) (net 5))
 (segment (start 249.5804 103.251) (end 251.079 104.7496) (width 0.762) (layer F.Cu) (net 5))
 (segment (start 232.918 133.5151) (end 239.9792 133.5151) (width 0.762) (layer F.Cu) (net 5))
 (segment (start 232.7783 124.4092) (end 231.0892 126.0983) (width 0.762) (layer F.Cu) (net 5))
 (segment (start 231.0892 126.0983) (end 231.0892 131.6863) (width 0.762) (layer F.Cu) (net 5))
 (segment (start 231.0892 131.6863) (end 232.918 133.5151) (width 0.762) (layer F.Cu) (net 5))
 (segment (start 239.9792 133.5151) (end 242.05438 131.43992) (width 0.762) (layer F.Cu) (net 5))
 (segment (start 242.05438 131.43992) (end 242.05438 130.1877) (width 0.762) (layer F.Cu) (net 5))
 (segment (start 233.73588 124.4092) (end 232.7783 124.4092) (width 0.762) (layer F.Cu) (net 5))
 (segment (start 222.5675 108.3945) (end 222.9485 108.3945) (width 0.762) (layer F.Cu) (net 5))
 (segment (start 245.427502 97.790002) (end 248.3485 100.711) (width 0.762) (layer F.Cu) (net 5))
 (segment (start 233.552998 97.790002) (end 245.427502 97.790002) (width 0.762) (layer F.Cu) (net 5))
 (segment (start 222.9485 108.3945) (end 233.552998 97.790002) (width 0.762) (layer F.Cu) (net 5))
 (segment (start 248.3485 100.711) (end 248.3485 103.251) (width 0.762) (layer F.Cu) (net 5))
 (segment (start 210.058 105.8545) (end 207.4545 105.8545) (width 0.254) (layer F.Cu) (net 13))
 (segment (start 250.952 124.809) (end 251.8598 124.809) (width 0.254) (layer F.Cu) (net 2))
 (segment (start 214.9348 100.9777) (end 217.678 98.2345) (width 0.254) (layer B.Cu) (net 2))
 (segment (start 214.9348 107.1372) (end 214.9348 100.9777) (width 0.254) (layer B.Cu) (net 2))
 (segment (start 212.1408 109.9312) (end 214.9348 107.1372) (width 0.254) (layer B.Cu) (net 2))
 (segment (start 210.0834 109.9312) (end 212.1408 109.9312) (width 0.254) (layer B.Cu) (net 2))
 (segment (start 209.0674 110.9472) (end 210.0834 109.9312) (width 0.254) (layer B.Cu) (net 2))
 (via (at 209.0674 110.9472) (size 0.889) (layers F.Cu B.Cu) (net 2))
 (segment (start 209.0674 125.6792) (end 209.0674 110.9472) (width 0.254) (layer F.Cu) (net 2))
 (segment (start 222.1738 138.7856) (end 209.0674 125.6792) (width 0.254) (layer F.Cu) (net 2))
 (segment (start 244.3226 138.7856) (end 222.1738 138.7856) (width 0.254) (layer F.Cu) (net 2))
 (segment (start 253.1872 129.921) (end 244.3226 138.7856) (width 0.254) (layer F.Cu) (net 2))
 (segment (start 253.1872 126.1364) (end 253.1872 129.921) (width 0.254) (layer F.Cu) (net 2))
 (segment (start 251.8598 124.809) (end 253.1872 126.1364) (width 0.254) (layer F.Cu) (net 2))
 (segment (start 215.9508 117.9068) (end 215.9508 120.7008) (width 0.254) (layer F.Cu) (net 9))
 (segment (start 236.0803 100.7745) (end 224.7392 112.1156) (width 0.254) (layer F.Cu) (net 9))
 (segment (start 224.7392 112.1156) (end 224.7392 119.9388) (width 0.254) (layer F.Cu) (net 9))
 (segment (start 215.9508 117.9068) (end 215.9508 102.5017) (width 0.254) (layer F.Cu) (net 9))
 (segment (start 217.678 100.7745) (end 215.9508 102.5017) (width 0.254) (layer F.Cu) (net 9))
 (segment (start 236.0803 100.7745) (end 237.8075 100.7745) (width 0.254) (layer F.Cu) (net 9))
 (segment (start 224.7392 122.174) (end 224.7392 119.9388) (width 0.254) (layer F.Cu) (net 9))
 (segment (start 221.996 124.9172) (end 224.7392 122.174) (width 0.254) (layer F.Cu) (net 9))
 (segment (start 220.1672 124.9172) (end 221.996 124.9172) (width 0.254) (layer F.Cu) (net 9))
 (segment (start 215.9508 120.7008) (end 220.1672 124.9172) (width 0.254) (layer F.Cu) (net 9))
 (segment (start 237.8075 103.3145) (end 235.4199 103.3145) (width 0.254) (layer F.Cu) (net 8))
 (segment (start 219.3925 103.3145) (end 217.678 103.3145) (width 0.254) (layer F.Cu) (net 8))
 (segment (start 220.6244 104.5464) (end 219.3925 103.3145) (width 0.254) (layer F.Cu) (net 8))
 (segment (start 220.6244 120.0912) (end 220.6244 104.5464) (width 0.254) (layer F.Cu) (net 8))
 (segment (start 220.98 120.4468) (end 220.6244 120.0912) (width 0.254) (layer F.Cu) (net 8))
 (via (at 220.98 120.4468) (size 0.889) (layers F.Cu B.Cu) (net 8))
 (segment (start 226.2124 120.4468) (end 220.98 120.4468) (width 0.254) (layer B.Cu) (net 8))
 (segment (start 226.8728 121.1072) (end 226.2124 120.4468) (width 0.254) (layer B.Cu) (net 8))
 (via (at 226.8728 121.1072) (size 0.889) (layers F.Cu B.Cu) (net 8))
 (segment (start 226.8728 111.8616) (end 226.8728 121.1072) (width 0.254) (layer F.Cu) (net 8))
 (segment (start 235.4199 103.3145) (end 226.8728 111.8616) (width 0.254) (layer F.Cu) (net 8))
 (segment (start 237.8075 105.8545) (end 237.0455 105.8545) (width 0.254) (layer F.Cu) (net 7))
 (segment (start 219.4052 107.5817) (end 217.678 105.8545) (width 0.254) (layer F.Cu) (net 7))
 (segment (start 219.4052 120.8024) (end 219.4052 107.5817) (width 0.254) (layer F.Cu) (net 7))
 (segment (start 218.7956 121.412) (end 219.4052 120.8024) (width 0.254) (layer F.Cu) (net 7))
 (via (at 218.7956 121.412) (size 0.889) (layers F.Cu B.Cu) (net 7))
 (segment (start 218.948 121.412) (end 218.7956 121.412) (width 0.254) (layer B.Cu) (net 7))
 (segment (start 219.9132 122.3772) (end 218.948 121.412) (width 0.254) (layer B.Cu) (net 7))
 (segment (start 227.6348 122.3772) (end 219.9132 122.3772) (width 0.254) (layer B.Cu) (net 7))
 (segment (start 228.8032 123.5456) (end 227.6348 122.3772) (width 0.254) (layer B.Cu) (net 7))
 (via (at 228.8032 123.5456) (size 0.889) (layers F.Cu B.Cu) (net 7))
 (segment (start 228.8032 114.0968) (end 228.8032 123.5456) (width 0.254) (layer F.Cu) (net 7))
 (segment (start 237.0455 105.8545) (end 228.8032 114.0968) (width 0.254) (layer F.Cu) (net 7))
 (segment (start 248.3485 109.4105) (end 248.3485 114.6683) (width 0.762) (layer F.Cu) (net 6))
 (segment (start 242.18138 120.83542) (end 242.18138 124.2822) (width 0.762) (layer F.Cu) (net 6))
 (segment (start 248.3485 114.6683) (end 242.18138 120.83542) (width 0.762) (layer F.Cu) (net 6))
 (segment (start 233.73588 130.2512) (end 233.73588 130.62458) (width 0.762) (layer F.Cu) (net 6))
 (segment (start 233.73588 130.62458) (end 235.5088 132.3975) (width 0.762) (layer F.Cu) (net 6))
 (segment (start 235.5088 132.3975) (end 239.268 132.3975) (width 0.762) (layer F.Cu) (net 6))
 (segment (start 239.268 132.3975) (end 239.776 131.8895) (width 0.762) (layer F.Cu) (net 6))
 (segment (start 239.776 131.8895) (end 239.776 126.68758) (width 0.762) (layer F.Cu) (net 6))
 (segment (start 239.776 126.68758) (end 242.18138 124.2822) (width 0.762) (layer F.Cu) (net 6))
 (segment (start 222.5675 110.9345) (end 223.52 110.9345) (width 0.762) (layer F.Cu) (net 6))
 (segment (start 240.538 99.06) (end 248.3485 106.8705) (width 0.762) (layer F.Cu) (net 6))
 (segment (start 235.3945 99.06) (end 240.538 99.06) (width 0.762) (layer F.Cu) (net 6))
 (segment (start 223.52 110.9345) (end 235.3945 99.06) (width 0.762) (layer F.Cu) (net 6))
 (segment (start 248.3485 106.8705) (end 248.3485 109.4105) (width 0.762) (layer F.Cu) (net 6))
 (segment (start 219.583 83.439) (end 216.4715 83.439) (width 0.254) (layer F.Cu) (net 12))
 (segment (start 215.0745 93.091) (end 217.678 95.6945) (width 0.254) (layer F.Cu) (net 12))
 (segment (start 215.0745 84.836) (end 215.0745 93.091) (width 0.254) (layer F.Cu) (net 12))
 (segment (start 216.4715 83.439) (end 215.0745 84.836) (width 0.254) (layer F.Cu) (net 12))
 (segment (start 210.058 103.3145) (end 207.391 103.3145) (width 0.254) (layer F.Cu) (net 14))
 (segment (start 205.9305 105.8545) (end 205.9305 109.9185) (width 0.254) (layer F.Cu) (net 11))
 (segment (start 207.4545 123.7615) (end 204.978 126.238) (width 0.254) (layer F.Cu) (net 11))
 (segment (start 207.4545 111.4425) (end 207.4545 123.7615) (width 0.254) (layer F.Cu) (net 11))
 (segment (start 205.9305 109.9185) (end 207.4545 111.4425) (width 0.254) (layer F.Cu) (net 11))
 (segment (start 205.867 103.3145) (end 204.851 103.3145) (width 0.254) (layer F.Cu) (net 10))
 (segment (start 203.3905 122.1105) (end 204.978 123.698) (width 0.254) (layer F.Cu) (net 10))
 (segment (start 203.3905 104.775) (end 203.3905 122.1105) (width 0.254) (layer F.Cu) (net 10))
 (segment (start 204.851 103.3145) (end 203.3905 104.775) (width 0.254) (layer F.Cu) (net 10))
 (segment (start 250.317 135.6868) (end 249.1232 135.6868) (width 0.254) (layer F.Cu) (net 15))
 (segment (start 201.0918 97.0407) (end 210.058 88.0745) (width 0.254) (layer F.Cu) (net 15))
 (segment (start 201.0918 137.2108) (end 201.0918 97.0407) (width 0.254) (layer F.Cu) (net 15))
 (segment (start 205.359 141.478) (end 201.0918 137.2108) (width 0.254) (layer F.Cu) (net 15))
 (segment (start 243.332 141.478) (end 205.359 141.478) (width 0.254) (layer F.Cu) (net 15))
 (segment (start 249.1232 135.6868) (end 243.332 141.478) (width 0.254) (layer F.Cu) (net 15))
 (segment (start 238.8362 135.5852) (end 232.0798 135.5852) (width 0.254) (layer F.Cu) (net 16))
 (segment (start 213.868 94.4245) (end 210.058 90.6145) (width 0.254) (layer F.Cu) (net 16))
 (segment (start 213.868 122.1232) (end 213.868 94.4245) (width 0.254) (layer F.Cu) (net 16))
 (segment (start 218.9226 127.1778) (end 213.868 122.1232) (width 0.254) (layer F.Cu) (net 16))
 (segment (start 223.6724 127.1778) (end 218.9226 127.1778) (width 0.254) (layer F.Cu) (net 16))
 (segment (start 232.0798 135.5852) (end 223.6724 127.1778) (width 0.254) (layer F.Cu) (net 16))
 (segment (start 227.6094 135.636) (end 223.3168 135.636) (width 0.254) (layer F.Cu) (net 17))
 (segment (start 212.09 95.1865) (end 210.058 93.1545) (width 0.254) (layer F.Cu) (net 17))
 (segment (start 212.09 124.4092) (end 212.09 95.1865) (width 0.254) (layer F.Cu) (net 17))
 (segment (start 223.3168 135.636) (end 212.09 124.4092) (width 0.254) (layer F.Cu) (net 17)))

